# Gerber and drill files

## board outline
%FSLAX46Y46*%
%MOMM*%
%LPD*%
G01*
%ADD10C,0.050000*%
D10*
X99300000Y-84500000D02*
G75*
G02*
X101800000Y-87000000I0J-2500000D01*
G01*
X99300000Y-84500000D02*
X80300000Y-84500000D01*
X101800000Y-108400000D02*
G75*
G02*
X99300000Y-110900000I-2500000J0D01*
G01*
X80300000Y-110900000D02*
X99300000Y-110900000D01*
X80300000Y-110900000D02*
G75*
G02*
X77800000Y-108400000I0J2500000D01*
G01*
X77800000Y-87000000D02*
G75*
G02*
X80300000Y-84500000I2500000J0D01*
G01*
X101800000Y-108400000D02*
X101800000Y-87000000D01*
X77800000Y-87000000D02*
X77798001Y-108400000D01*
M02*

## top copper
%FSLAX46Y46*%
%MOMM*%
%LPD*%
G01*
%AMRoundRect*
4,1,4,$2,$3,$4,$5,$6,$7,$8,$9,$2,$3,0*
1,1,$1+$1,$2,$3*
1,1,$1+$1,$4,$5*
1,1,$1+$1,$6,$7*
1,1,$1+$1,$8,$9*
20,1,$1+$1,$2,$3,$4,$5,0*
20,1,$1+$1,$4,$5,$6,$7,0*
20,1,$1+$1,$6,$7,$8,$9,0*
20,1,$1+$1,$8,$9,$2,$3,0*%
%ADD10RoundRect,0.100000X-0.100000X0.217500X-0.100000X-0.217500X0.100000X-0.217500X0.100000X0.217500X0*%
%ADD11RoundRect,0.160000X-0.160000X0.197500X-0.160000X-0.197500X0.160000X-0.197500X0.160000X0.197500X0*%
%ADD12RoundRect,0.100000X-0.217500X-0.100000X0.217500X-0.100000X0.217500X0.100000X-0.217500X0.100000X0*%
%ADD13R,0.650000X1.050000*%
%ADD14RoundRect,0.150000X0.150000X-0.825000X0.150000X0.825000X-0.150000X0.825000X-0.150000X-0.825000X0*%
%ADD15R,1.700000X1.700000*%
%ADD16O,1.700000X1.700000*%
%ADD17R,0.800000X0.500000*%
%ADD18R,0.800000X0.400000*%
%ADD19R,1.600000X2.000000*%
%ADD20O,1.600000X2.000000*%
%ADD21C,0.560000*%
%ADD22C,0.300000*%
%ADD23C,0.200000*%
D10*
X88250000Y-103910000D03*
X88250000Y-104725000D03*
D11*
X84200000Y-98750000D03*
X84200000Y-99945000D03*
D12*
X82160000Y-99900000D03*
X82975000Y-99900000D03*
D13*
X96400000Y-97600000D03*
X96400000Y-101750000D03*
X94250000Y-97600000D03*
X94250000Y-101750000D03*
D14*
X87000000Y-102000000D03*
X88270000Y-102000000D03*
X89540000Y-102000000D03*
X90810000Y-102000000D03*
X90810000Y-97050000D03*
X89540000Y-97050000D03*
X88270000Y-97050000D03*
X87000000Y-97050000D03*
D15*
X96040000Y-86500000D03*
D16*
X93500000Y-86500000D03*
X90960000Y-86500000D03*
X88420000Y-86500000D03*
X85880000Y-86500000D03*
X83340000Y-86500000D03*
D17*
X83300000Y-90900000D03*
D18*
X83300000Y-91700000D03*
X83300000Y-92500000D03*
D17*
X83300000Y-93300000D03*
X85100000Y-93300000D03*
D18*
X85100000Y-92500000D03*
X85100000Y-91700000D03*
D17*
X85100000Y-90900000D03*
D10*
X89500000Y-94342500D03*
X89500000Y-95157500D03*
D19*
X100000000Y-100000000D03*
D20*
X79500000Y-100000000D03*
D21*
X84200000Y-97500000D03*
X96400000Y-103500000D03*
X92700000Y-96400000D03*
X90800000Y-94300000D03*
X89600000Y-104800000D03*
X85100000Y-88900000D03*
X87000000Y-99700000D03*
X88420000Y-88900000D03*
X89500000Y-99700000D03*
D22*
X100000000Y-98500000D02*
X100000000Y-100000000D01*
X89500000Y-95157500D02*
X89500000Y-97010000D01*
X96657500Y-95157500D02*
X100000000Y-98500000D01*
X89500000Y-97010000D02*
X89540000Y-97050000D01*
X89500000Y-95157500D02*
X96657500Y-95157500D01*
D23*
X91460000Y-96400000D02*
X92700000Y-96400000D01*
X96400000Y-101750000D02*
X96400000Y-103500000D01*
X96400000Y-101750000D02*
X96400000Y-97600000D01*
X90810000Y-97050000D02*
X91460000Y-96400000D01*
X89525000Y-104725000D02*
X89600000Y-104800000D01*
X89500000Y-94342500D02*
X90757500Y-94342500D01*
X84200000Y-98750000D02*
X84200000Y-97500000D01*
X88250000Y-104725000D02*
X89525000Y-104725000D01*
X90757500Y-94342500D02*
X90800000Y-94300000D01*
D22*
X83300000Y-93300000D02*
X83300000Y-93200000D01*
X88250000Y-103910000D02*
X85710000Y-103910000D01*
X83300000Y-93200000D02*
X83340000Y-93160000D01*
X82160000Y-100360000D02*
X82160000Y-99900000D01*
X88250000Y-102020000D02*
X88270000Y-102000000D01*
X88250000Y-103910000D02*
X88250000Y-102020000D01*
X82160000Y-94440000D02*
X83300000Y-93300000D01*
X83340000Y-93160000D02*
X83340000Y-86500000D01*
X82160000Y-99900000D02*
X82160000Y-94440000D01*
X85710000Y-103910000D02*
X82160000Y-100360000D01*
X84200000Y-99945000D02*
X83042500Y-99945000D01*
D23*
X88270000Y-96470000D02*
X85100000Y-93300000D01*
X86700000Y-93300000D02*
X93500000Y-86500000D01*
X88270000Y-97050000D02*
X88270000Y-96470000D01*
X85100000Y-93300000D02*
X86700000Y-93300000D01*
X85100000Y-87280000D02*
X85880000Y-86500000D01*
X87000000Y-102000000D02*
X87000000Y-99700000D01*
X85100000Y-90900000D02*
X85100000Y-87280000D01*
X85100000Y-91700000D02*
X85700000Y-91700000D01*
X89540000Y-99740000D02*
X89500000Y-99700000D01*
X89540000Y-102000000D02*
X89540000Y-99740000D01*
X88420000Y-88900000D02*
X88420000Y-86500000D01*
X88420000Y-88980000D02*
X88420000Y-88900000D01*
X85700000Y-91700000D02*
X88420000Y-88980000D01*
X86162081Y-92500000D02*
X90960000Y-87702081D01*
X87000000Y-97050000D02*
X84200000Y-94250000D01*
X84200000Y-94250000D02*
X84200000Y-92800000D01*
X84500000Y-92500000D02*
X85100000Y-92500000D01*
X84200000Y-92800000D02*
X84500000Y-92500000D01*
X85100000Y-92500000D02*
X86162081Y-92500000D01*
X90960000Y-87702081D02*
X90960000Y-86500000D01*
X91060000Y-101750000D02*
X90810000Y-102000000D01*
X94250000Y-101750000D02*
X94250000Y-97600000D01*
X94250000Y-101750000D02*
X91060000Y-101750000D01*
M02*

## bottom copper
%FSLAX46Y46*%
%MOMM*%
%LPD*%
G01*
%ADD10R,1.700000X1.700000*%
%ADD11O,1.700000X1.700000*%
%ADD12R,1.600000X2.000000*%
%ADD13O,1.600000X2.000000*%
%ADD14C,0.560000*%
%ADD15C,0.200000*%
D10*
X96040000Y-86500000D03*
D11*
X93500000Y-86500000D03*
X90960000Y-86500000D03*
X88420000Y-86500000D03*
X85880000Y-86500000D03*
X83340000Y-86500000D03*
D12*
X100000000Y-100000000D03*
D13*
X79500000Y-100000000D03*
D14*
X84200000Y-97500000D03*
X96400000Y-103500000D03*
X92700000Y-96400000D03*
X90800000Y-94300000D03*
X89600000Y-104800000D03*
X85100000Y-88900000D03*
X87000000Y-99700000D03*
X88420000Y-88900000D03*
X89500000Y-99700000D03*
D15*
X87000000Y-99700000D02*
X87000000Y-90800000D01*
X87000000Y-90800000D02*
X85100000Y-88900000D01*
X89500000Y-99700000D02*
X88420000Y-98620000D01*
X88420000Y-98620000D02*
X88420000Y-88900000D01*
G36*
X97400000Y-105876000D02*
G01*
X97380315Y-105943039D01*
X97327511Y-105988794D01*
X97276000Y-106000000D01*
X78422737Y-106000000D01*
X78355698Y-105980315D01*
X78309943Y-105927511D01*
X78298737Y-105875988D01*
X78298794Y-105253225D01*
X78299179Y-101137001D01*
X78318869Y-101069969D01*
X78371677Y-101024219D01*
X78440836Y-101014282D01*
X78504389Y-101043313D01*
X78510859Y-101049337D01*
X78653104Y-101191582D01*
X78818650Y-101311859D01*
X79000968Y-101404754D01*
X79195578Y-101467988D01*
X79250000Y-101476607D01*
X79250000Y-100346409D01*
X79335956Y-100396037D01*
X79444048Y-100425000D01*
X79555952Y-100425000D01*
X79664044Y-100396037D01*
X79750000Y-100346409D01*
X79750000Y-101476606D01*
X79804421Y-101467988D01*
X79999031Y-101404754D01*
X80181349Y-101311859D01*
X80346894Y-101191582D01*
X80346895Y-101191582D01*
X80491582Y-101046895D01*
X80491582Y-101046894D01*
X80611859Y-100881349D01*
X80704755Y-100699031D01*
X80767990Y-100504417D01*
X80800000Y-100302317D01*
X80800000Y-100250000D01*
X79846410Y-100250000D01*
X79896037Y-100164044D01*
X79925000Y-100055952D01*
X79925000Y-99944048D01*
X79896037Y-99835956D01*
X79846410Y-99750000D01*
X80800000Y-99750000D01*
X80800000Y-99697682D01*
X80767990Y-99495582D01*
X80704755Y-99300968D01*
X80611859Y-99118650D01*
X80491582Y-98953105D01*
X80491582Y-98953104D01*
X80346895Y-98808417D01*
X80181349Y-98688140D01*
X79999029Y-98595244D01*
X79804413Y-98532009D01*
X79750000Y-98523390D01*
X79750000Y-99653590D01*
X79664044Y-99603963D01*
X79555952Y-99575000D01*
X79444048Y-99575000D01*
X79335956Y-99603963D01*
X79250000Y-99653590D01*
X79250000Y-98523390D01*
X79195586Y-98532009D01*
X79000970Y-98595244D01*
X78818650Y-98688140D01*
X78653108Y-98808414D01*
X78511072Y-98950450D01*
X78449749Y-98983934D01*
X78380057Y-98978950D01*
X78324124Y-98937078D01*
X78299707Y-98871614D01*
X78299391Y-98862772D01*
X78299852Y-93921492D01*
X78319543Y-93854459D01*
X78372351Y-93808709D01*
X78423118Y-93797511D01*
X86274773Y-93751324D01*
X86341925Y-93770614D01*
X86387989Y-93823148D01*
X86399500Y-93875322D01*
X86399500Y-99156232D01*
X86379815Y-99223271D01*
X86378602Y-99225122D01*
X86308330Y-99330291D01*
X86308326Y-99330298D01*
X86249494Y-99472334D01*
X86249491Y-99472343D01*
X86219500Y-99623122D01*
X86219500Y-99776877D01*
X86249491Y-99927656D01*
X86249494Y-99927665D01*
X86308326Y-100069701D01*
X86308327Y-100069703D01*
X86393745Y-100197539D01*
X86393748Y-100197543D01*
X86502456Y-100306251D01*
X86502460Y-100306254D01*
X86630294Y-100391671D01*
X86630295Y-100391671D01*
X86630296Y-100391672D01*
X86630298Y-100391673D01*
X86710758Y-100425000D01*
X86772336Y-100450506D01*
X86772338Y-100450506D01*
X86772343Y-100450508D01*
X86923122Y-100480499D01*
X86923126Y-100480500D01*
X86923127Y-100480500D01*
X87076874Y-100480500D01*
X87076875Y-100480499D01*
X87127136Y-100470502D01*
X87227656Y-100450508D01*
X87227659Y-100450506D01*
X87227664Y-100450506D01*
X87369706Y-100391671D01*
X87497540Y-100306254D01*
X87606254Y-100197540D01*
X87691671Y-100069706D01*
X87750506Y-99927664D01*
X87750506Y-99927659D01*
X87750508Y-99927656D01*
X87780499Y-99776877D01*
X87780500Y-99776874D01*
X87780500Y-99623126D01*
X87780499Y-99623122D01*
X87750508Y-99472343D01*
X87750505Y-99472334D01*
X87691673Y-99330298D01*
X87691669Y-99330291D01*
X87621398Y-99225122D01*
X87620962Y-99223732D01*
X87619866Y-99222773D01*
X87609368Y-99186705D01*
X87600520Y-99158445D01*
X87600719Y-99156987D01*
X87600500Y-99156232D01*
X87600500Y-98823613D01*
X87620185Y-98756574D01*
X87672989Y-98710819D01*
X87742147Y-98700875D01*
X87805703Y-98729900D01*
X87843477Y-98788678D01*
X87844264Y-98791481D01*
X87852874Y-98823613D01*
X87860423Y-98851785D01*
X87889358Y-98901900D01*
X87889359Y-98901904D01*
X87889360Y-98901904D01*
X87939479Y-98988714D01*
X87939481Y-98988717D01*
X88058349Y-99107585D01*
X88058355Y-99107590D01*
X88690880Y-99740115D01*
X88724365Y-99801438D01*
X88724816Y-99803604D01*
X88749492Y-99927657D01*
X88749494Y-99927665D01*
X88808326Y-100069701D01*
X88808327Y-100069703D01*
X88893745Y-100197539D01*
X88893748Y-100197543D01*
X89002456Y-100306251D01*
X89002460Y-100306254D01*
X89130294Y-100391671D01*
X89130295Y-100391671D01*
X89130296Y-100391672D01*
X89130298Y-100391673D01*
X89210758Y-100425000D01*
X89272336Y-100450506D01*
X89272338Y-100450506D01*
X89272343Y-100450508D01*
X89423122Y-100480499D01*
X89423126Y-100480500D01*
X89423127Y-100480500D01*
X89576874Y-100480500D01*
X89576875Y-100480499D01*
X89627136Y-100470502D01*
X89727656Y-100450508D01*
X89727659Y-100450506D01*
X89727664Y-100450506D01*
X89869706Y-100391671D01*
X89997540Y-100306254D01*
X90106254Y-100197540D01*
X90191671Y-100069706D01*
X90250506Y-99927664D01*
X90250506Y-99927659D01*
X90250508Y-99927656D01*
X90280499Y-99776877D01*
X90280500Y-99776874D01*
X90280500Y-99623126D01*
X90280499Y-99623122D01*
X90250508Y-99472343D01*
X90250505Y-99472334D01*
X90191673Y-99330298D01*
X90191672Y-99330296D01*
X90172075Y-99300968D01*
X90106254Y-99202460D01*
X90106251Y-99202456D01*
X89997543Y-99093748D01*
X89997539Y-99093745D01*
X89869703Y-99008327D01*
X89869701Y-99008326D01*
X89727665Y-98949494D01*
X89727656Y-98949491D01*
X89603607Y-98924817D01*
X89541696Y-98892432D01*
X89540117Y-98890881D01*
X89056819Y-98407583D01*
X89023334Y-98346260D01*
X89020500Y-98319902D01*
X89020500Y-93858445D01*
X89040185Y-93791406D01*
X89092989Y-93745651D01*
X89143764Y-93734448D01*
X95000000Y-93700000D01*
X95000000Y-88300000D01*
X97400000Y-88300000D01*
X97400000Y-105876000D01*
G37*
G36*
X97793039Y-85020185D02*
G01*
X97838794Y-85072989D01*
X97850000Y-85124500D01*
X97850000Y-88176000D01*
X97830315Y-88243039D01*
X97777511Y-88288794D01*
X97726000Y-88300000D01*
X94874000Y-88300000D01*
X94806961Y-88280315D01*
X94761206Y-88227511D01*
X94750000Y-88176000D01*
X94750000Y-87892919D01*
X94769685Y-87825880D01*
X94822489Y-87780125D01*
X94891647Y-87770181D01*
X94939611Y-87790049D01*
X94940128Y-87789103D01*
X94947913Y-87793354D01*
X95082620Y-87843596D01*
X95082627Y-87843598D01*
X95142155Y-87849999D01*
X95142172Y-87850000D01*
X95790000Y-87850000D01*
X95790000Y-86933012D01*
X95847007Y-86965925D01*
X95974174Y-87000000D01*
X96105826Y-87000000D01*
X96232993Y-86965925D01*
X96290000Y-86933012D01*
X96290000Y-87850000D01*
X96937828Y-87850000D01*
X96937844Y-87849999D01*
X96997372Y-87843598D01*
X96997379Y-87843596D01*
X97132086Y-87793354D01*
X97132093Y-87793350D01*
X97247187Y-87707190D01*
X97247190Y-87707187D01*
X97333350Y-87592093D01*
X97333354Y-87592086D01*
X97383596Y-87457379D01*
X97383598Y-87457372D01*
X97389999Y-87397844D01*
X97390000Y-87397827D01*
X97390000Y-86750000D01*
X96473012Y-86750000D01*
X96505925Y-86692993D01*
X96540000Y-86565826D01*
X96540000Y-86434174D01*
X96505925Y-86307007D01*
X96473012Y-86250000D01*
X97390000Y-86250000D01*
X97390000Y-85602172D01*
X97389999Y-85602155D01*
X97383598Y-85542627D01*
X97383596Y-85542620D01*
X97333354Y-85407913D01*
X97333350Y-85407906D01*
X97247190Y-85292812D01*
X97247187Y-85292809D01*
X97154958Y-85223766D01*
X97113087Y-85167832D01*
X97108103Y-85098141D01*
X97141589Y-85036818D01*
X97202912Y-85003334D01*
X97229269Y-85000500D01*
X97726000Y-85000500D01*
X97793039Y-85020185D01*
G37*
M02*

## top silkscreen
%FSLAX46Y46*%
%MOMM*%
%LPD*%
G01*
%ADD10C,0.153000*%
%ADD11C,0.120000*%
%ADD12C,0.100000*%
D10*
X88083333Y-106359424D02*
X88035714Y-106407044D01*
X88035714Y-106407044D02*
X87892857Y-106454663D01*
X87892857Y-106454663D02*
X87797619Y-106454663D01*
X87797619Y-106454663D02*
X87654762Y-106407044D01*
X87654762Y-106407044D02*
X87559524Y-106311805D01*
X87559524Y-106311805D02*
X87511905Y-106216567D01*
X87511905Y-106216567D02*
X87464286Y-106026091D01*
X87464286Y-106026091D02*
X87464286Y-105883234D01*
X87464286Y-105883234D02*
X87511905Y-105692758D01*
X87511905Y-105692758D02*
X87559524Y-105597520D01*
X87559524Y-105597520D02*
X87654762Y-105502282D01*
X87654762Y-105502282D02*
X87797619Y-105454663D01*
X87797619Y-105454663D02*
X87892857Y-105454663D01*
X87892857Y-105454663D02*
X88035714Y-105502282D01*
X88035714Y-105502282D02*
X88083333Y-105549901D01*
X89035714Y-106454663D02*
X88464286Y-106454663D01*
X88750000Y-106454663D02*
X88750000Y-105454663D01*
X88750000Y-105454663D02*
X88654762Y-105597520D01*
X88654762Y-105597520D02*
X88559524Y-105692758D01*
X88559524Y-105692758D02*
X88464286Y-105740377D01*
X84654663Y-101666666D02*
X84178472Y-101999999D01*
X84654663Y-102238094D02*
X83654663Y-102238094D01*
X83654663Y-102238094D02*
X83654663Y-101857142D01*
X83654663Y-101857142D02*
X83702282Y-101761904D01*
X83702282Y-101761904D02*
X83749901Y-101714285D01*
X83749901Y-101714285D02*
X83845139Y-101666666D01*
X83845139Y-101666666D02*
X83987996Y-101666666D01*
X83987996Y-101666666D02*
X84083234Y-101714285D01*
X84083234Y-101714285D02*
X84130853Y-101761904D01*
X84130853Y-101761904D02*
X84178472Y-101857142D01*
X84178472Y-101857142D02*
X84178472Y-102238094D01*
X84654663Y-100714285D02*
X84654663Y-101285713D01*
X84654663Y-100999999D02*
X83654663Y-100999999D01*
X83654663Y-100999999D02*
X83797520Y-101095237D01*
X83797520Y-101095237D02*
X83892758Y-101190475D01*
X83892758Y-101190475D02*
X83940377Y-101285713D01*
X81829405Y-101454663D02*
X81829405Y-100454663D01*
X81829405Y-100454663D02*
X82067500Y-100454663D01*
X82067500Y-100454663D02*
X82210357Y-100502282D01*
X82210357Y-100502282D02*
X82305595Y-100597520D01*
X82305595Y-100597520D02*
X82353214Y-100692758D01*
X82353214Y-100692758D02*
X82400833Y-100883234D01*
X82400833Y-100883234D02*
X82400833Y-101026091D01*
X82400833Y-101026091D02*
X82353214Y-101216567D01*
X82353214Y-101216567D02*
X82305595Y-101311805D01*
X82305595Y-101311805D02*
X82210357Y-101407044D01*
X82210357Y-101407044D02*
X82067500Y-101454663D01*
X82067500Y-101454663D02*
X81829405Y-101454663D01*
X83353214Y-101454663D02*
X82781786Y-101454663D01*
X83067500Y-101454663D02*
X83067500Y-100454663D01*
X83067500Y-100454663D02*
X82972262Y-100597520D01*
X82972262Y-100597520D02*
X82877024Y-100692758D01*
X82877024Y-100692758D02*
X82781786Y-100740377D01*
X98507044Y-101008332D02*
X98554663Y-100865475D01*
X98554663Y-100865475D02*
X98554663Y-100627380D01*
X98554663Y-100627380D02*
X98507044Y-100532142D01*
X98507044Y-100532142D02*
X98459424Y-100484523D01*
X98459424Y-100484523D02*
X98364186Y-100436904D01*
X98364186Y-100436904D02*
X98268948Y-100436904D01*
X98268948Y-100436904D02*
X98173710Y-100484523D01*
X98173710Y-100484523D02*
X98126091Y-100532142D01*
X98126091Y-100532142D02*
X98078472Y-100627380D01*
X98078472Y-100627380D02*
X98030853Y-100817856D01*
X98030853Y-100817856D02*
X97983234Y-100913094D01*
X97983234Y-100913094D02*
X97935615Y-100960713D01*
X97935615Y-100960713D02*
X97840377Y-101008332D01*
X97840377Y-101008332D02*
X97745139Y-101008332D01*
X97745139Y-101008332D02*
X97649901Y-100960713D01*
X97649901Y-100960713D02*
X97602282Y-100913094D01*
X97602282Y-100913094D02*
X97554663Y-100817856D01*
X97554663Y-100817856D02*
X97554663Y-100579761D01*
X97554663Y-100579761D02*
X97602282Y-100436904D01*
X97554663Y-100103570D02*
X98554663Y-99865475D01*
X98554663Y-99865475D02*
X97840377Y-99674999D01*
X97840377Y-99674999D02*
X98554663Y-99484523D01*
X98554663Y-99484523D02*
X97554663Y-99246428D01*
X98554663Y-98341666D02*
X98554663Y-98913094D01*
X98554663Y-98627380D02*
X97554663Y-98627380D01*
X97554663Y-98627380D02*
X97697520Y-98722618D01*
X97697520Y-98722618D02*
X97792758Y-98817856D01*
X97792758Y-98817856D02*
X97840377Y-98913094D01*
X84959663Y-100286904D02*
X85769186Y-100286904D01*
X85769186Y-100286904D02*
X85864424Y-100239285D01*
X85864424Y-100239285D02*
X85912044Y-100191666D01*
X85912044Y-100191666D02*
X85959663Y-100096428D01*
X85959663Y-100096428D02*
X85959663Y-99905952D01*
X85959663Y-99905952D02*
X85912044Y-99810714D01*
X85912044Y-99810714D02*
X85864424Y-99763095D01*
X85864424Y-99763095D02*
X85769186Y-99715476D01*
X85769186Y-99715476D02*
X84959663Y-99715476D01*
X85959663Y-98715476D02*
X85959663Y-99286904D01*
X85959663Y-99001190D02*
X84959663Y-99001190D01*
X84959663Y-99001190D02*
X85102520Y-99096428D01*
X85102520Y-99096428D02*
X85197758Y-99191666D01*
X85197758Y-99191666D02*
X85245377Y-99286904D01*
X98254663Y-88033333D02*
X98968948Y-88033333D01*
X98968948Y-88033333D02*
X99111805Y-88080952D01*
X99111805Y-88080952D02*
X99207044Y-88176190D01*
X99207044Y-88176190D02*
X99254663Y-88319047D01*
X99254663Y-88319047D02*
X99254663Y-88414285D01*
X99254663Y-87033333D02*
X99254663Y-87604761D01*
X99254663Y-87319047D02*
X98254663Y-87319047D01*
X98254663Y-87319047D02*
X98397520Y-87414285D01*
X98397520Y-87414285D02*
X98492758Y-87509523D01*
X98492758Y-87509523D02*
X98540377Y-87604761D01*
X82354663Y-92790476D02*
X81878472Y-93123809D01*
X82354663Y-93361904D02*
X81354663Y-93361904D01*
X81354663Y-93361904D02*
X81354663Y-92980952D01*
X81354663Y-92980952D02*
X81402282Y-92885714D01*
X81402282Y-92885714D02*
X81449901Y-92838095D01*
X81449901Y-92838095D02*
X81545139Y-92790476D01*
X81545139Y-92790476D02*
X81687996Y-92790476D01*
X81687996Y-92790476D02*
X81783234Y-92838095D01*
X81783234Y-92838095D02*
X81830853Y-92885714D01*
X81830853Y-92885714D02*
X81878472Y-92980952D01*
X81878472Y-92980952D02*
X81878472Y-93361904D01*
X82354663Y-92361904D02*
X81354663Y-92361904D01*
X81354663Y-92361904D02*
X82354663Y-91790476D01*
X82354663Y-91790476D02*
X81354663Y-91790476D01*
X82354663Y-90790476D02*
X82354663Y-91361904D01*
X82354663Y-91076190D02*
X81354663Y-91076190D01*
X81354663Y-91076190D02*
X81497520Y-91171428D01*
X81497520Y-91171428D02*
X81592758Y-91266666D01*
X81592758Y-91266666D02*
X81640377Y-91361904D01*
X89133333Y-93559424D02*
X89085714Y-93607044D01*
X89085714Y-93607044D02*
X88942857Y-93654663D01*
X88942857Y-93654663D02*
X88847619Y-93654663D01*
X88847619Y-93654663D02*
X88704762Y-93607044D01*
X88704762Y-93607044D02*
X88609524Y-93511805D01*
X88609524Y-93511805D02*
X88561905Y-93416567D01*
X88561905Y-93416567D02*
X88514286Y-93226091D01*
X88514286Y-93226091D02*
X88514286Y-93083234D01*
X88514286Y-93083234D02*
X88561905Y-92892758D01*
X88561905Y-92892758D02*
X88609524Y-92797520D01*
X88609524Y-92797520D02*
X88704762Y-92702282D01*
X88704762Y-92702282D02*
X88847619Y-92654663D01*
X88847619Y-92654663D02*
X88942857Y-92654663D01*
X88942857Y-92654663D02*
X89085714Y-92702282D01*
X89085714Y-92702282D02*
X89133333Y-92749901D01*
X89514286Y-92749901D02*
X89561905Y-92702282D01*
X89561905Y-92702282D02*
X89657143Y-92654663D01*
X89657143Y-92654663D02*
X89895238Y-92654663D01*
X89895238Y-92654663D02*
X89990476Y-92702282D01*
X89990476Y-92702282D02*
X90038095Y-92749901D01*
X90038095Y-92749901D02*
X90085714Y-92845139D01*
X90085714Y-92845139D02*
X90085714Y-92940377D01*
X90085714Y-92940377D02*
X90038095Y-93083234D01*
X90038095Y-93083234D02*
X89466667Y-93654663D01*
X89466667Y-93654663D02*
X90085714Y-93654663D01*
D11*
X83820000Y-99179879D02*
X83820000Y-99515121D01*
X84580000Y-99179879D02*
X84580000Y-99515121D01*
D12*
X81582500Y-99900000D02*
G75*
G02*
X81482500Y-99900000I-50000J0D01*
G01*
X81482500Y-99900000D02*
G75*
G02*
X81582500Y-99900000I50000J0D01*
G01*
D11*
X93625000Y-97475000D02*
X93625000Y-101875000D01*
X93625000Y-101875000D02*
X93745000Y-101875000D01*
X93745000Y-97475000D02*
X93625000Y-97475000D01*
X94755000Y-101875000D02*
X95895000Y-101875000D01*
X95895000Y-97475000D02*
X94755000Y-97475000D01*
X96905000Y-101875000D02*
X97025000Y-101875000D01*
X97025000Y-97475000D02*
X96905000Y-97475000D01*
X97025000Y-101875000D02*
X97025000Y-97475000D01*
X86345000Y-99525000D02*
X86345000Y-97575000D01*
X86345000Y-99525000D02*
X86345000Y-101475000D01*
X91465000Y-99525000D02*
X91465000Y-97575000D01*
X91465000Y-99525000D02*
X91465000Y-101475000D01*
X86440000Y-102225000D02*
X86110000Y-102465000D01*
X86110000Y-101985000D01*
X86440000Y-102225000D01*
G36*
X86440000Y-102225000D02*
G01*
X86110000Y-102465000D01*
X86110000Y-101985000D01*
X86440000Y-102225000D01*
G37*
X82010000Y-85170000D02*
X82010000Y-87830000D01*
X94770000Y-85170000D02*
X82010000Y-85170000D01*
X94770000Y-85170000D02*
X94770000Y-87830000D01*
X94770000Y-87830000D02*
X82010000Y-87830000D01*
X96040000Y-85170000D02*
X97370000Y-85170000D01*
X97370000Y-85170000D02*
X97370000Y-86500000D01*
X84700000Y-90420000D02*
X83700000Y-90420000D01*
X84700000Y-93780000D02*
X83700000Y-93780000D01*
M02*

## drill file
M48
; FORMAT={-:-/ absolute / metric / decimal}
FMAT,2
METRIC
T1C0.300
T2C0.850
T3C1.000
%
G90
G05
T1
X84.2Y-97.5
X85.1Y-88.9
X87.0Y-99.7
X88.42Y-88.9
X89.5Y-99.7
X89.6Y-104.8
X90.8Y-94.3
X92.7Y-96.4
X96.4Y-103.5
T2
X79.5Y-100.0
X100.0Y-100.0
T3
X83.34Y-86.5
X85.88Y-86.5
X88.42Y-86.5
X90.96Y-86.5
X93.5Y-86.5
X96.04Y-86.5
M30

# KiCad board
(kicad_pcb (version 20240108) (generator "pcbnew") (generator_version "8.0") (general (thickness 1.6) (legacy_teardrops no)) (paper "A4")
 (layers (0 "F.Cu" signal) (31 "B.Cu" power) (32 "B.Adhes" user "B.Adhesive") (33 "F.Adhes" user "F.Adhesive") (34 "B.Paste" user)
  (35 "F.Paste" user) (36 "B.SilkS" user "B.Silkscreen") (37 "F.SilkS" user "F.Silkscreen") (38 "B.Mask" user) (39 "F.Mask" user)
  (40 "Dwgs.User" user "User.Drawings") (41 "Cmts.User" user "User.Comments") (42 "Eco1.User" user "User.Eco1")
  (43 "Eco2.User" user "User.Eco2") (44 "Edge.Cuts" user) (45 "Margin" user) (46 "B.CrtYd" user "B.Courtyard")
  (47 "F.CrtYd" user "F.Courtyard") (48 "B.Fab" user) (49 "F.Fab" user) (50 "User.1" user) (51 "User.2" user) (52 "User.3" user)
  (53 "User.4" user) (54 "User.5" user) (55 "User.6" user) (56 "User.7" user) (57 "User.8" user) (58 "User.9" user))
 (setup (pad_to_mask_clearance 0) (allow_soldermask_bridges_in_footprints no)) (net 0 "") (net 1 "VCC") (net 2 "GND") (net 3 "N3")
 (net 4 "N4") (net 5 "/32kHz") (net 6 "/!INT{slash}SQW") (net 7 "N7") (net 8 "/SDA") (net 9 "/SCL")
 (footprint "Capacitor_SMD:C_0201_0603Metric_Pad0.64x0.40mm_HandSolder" (layer "F.Cu") (at 88.25 104.3175 -90)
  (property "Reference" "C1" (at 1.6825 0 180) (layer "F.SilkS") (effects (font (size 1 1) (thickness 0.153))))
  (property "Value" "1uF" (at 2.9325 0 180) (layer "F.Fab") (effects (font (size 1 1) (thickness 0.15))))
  (pad "" smd roundrect (at -0.4325 0 270) (size 0.458 0.36) (layers "F.Paste") (roundrect_rratio 0.25))
  (pad "" smd roundrect (at 0.4325 0 270) (size 0.458 0.36) (layers "F.Paste") (roundrect_rratio 0.25))
  (pad "1" smd roundrect (at -0.4075 0 270) (size 0.635 0.4) (layers "F.Cu" "F.Mask") (roundrect_rratio 0.25) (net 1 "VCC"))
  (pad "2" smd roundrect (at 0.4075 0 270) (size 0.635 0.4) (layers "F.Cu" "F.Mask") (roundrect_rratio 0.25) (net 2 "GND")))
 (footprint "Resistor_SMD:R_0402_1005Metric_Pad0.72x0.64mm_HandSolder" (layer "F.Cu") (at 84.2 99.3475 -90)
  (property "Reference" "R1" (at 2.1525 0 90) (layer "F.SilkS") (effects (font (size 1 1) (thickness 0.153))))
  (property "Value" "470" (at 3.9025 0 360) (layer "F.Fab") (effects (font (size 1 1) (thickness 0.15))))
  (fp_line (start -0.167621 0.38) (end 0.167621 0.38) (stroke (width 0.12) (type solid)) (layer "F.SilkS"))
  (fp_line (start -0.167621 -0.38) (end 0.167621 -0.38) (stroke (width 0.12) (type solid)) (layer "F.SilkS"))
  (pad "1" smd roundrect (at -0.5975 0 270) (size 0.715 0.64) (layers "F.Cu" "F.Paste" "F.Mask") (roundrect_rratio 0.25) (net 2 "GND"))
  (pad "2" smd roundrect (at 0.5975 0 270) (size 0.715 0.64) (layers "F.Cu" "F.Paste" "F.Mask") (roundrect_rratio 0.25) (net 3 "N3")))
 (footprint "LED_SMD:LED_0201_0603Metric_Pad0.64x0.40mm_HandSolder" (layer "F.Cu") (at 82.5675 99.9)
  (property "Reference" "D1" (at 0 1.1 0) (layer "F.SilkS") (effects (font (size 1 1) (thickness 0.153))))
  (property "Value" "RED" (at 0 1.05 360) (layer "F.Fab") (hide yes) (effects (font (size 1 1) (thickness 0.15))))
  (fp_circle (center -1.035 0) (end -0.985 0) (stroke (width 0.1) (type solid)) (fill none) (layer "F.SilkS"))
  (pad "" smd roundrect (at -0.4325 0) (size 0.458 0.36) (layers "F.Paste") (roundrect_rratio 0.25))
  (pad "" smd roundrect (at 0.4325 0) (size 0.458 0.36) (layers "F.Paste") (roundrect_rratio 0.25))
  (pad "1" smd roundrect (at -0.4075 0) (size 0.635 0.4) (layers "F.Cu" "F.Mask") (roundrect_rratio 0.25) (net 1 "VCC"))
  (pad "2" smd roundrect (at 0.4075 0) (size 0.635 0.4) (layers "F.Cu" "F.Mask") (roundrect_rratio 0.25) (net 3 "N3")))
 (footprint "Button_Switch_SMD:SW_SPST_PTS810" (layer "F.Cu") (at 95.325 99.675 -90)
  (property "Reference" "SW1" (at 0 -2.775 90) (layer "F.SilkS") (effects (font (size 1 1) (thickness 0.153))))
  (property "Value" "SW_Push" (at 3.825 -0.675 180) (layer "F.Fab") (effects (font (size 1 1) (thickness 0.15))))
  (fp_line (start -2.2 1.7) (end 2.2 1.7) (stroke (width 0.12) (type solid)) (layer "F.SilkS"))
  (fp_line (start 2.2 1.7) (end 2.2 1.58) (stroke (width 0.12) (type solid)) (layer "F.SilkS"))
  (fp_line (start -2.2 1.58) (end -2.2 1.7) (stroke (width 0.12) (type solid)) (layer "F.SilkS"))
  (fp_line (start 2.2 0.57) (end 2.2 -0.57) (stroke (width 0.12) (type solid)) (layer "F.SilkS"))
  (fp_line (start -2.2 -0.57) (end -2.2 0.57) (stroke (width 0.12) (type solid)) (layer "F.SilkS"))
  (fp_line (start 2.2 -1.58) (end 2.2 -1.7) (stroke (width 0.12) (type solid)) (layer "F.SilkS"))
  (fp_line (start -2.2 -1.7) (end -2.2 -1.58) (stroke (width 0.12) (type solid)) (layer "F.SilkS"))
  (fp_line (start 2.2 -1.7) (end -2.2 -1.7) (stroke (width 0.12) (type solid)) (layer "F.SilkS"))
  (pad "1" smd rect (at -2.075 -1.075 270) (size 1.05 0.65) (layers "F.Cu" "F.Paste" "F.Mask") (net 2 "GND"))
  (pad "1" smd rect (at 2.075 -1.075 270) (size 1.05 0.65) (layers "F.Cu" "F.Paste" "F.Mask") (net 2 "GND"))
  (pad "2" smd rect (at -2.075 1.075 270) (size 1.05 0.65) (layers "F.Cu" "F.Paste" "F.Mask") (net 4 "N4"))
  (pad "2" smd rect (at 2.075 1.075 270) (size 1.05 0.65) (layers "F.Cu" "F.Paste" "F.Mask") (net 4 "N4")))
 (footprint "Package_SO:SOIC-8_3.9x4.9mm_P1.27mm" (layer "F.Cu") (at 88.905 99.525 90)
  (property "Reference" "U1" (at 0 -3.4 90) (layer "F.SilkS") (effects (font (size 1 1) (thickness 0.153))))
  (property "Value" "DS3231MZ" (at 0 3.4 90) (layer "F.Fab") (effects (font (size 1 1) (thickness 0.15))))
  (fp_line (start 0 -2.56) (end 1.95 -2.56) (stroke (width 0.12) (type solid)) (layer "F.SilkS"))
  (fp_line (start 0 -2.56) (end -1.95 -2.56) (stroke (width 0.12) (type solid)) (layer "F.SilkS"))
  (fp_line (start 0 2.56) (end 1.95 2.56) (stroke (width 0.12) (type solid)) (layer "F.SilkS"))
  (fp_line (start 0 2.56) (end -1.95 2.56) (stroke (width 0.12) (type solid)) (layer "F.SilkS"))
  (fp_poly
   (pts (xy -2.7 -2.465) (xy -2.94 -2.795) (xy -2.46 -2.795) (xy -2.7 -2.465)) (stroke (width 0.12) (type solid)) (fill solid)
   (layer "F.SilkS"))
  (pad "1" smd roundrect (at -2.475 -1.905 90) (size 1.95 0.6) (layers "F.Cu" "F.Paste" "F.Mask") (roundrect_rratio 0.25) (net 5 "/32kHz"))
  (pad "2" smd roundrect (at -2.475 -0.635 90) (size 1.95 0.6) (layers "F.Cu" "F.Paste" "F.Mask") (roundrect_rratio 0.25) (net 1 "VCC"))
  (pad "3" smd roundrect (at -2.475 0.635 90) (size 1.95 0.6) (layers "F.Cu" "F.Paste" "F.Mask") (roundrect_rratio 0.25)
   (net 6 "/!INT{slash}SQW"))
  (pad "4" smd roundrect (at -2.475 1.905 90) (size 1.95 0.6) (layers "F.Cu" "F.Paste" "F.Mask") (roundrect_rratio 0.25) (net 4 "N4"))
  (pad "5" smd roundrect (at 2.475 1.905 90) (size 1.95 0.6) (layers "F.Cu" "F.Paste" "F.Mask") (roundrect_rratio 0.25) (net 2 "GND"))
  (pad "6" smd roundrect (at 2.475 0.635 90) (size 1.95 0.6) (layers "F.Cu" "F.Paste" "F.Mask") (roundrect_rratio 0.25) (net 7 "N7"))
  (pad "7" smd roundrect (at 2.475 -0.635 90) (size 1.95 0.6) (layers "F.Cu" "F.Paste" "F.Mask") (roundrect_rratio 0.25) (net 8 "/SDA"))
  (pad "8" smd roundrect (at 2.475 -1.905 90) (size 1.95 0.6) (layers "F.Cu" "F.Paste" "F.Mask") (roundrect_rratio 0.25) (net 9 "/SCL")))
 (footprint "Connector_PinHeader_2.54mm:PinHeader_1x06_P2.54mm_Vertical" (layer "F.Cu") (at 96.04 86.5 -90)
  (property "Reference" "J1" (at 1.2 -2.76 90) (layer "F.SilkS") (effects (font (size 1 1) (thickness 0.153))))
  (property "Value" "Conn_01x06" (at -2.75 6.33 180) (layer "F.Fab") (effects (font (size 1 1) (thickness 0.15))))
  (fp_line (start -1.33 14.03) (end 1.33 14.03) (stroke (width 0.12) (type solid)) (layer "F.SilkS"))
  (fp_line (start -1.33 1.27) (end -1.33 14.03) (stroke (width 0.12) (type solid)) (layer "F.SilkS"))
  (fp_line (start -1.33 1.27) (end 1.33 1.27) (stroke (width 0.12) (type solid)) (layer "F.SilkS"))
  (fp_line (start 1.33 1.27) (end 1.33 14.03) (stroke (width 0.12) (type solid)) (layer "F.SilkS"))
  (fp_line (start -1.33 0) (end -1.33 -1.33) (stroke (width 0.12) (type solid)) (layer "F.SilkS"))
  (fp_line (start -1.33 -1.33) (end 0 -1.33) (stroke (width 0.12) (type solid)) (layer "F.SilkS"))
  (pad "1" thru_hole rect (at 0 0 270) (size 1.7 1.7) (drill 1) (layers "*.Cu" "*.Mask") (remove_unused_layers no) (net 2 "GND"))
  (pad "2" thru_hole oval (at 0 2.54 270) (size 1.7 1.7) (drill 1) (layers "*.Cu" "*.Mask") (remove_unused_layers no) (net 8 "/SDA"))
  (pad "3" thru_hole oval (at 0 5.08 270) (size 1.7 1.7) (drill 1) (layers "*.Cu" "*.Mask") (remove_unused_layers no) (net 9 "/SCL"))
  (pad "4" thru_hole oval (at 0 7.62 270) (size 1.7 1.7) (drill 1) (layers "*.Cu" "*.Mask") (remove_unused_layers no)
   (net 6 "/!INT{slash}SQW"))
  (pad "5" thru_hole oval (at 0 10.16 270) (size 1.7 1.7) (drill 1) (layers "*.Cu" "*.Mask") (remove_unused_layers no) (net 5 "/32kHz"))
  (pad "6" thru_hole oval (at 0 12.7 270) (size 1.7 1.7) (drill 1) (layers "*.Cu" "*.Mask") (remove_unused_layers no) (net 1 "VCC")))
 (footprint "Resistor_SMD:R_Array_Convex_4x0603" (layer "F.Cu") (at 84.2 92.1)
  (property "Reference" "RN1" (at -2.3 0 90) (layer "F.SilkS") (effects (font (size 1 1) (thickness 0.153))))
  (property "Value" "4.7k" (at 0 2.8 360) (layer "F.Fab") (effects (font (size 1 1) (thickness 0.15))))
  (fp_line (start 0.5 -1.68) (end -0.5 -1.68) (stroke (width 0.12) (type solid)) (layer "F.SilkS"))
  (fp_line (start 0.5 1.68) (end -0.5 1.68) (stroke (width 0.12) (type solid)) (layer "F.SilkS"))
  (pad "1" smd rect (at -0.9 -1.2) (size 0.8 0.5) (layers "F.Cu" "F.Paste" "F.Mask") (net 1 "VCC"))
  (pad "2" smd rect (at -0.9 -0.4) (size 0.8 0.4) (layers "F.Cu" "F.Paste" "F.Mask") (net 1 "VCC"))
  (pad "3" smd rect (at -0.9 0.4) (size 0.8 0.4) (layers "F.Cu" "F.Paste" "F.Mask") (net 1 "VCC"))
  (pad "4" smd rect (at -0.9 1.2) (size 0.8 0.5) (layers "F.Cu" "F.Paste" "F.Mask") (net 1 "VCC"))
  (pad "5" smd rect (at 0.9 1.2) (size 0.8 0.5) (layers "F.Cu" "F.Paste" "F.Mask") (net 8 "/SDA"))
  (pad "6" smd rect (at 0.9 0.4) (size 0.8 0.4) (layers "F.Cu" "F.Paste" "F.Mask") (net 9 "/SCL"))
  (pad "7" smd rect (at 0.9 -0.4) (size 0.8 0.4) (layers "F.Cu" "F.Paste" "F.Mask") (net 6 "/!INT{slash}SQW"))
  (pad "8" smd rect (at 0.9 -1.2) (size 0.8 0.5) (layers "F.Cu" "F.Paste" "F.Mask") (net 5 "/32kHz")))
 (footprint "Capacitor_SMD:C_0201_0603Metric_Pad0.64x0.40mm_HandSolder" (layer "F.Cu") (at 89.5 94.75 -90)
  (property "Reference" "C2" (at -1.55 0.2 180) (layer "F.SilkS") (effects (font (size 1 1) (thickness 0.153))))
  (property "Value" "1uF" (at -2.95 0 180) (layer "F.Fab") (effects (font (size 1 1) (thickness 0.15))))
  (pad "" smd roundrect (at -0.4325 0 270) (size 0.458 0.36) (layers "F.Paste") (roundrect_rratio 0.25))
  (pad "" smd roundrect (at 0.4325 0 270) (size 0.458 0.36) (layers "F.Paste") (roundrect_rratio 0.25))
  (pad "1" smd roundrect (at -0.4075 0 270) (size 0.635 0.4) (layers "F.Cu" "F.Mask") (roundrect_rratio 0.25) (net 2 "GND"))
  (pad "2" smd roundrect (at 0.4075 0 270) (size 0.635 0.4) (layers "F.Cu" "F.Mask") (roundrect_rratio 0.25) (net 7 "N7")))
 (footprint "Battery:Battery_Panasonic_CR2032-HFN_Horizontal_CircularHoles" (layer "B.Cu") (at 100 100 180)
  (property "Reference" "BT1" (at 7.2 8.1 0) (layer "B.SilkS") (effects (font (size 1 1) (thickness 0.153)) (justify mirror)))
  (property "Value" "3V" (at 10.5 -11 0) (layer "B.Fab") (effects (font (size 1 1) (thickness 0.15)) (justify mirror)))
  (pad "1" thru_hole rect (at 0 0 180) (size 1.6 2) (drill 0.85) (layers "*.Cu" "*.Mask") (remove_unused_layers no) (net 7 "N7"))
  (pad "2" thru_hole oval (at 20.5 0 180) (size 1.6 2) (drill 0.85) (layers "*.Cu" "*.Mask") (remove_unused_layers no) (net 2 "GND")))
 (gr_arc (start 99.3 84.5) (mid 101.067767 85.232233) (end 101.8 87) (stroke (width 0.05) (type default)) (layer "Edge.Cuts"))
 (gr_line (start 99.3 84.5) (end 80.3 84.5) (stroke (width 0.05) (type default)) (layer "Edge.Cuts"))
 (gr_arc (start 101.8 108.4) (mid 101.067767 110.167767) (end 99.3 110.9) (stroke (width 0.05) (type default)) (layer "Edge.Cuts"))
 (gr_line (start 80.3 110.9) (end 99.3 110.9) (stroke (width 0.05) (type default)) (layer "Edge.Cuts"))
 (gr_arc (start 80.3 110.9) (mid 78.532233 110.167767) (end 77.8 108.4) (stroke (width 0.05) (type default)) (layer "Edge.Cuts"))
 (gr_arc (start 77.8 87) (mid 78.532233 85.232233) (end 80.3 84.5) (stroke (width 0.05) (type default)) (layer "Edge.Cuts"))
 (gr_line (start 101.8 108.4) (end 101.8 87) (stroke (width 0.05) (type default)) (layer "Edge.Cuts"))
 (gr_line (start 77.8 87) (end 77.798001 108.4) (stroke (width 0.05) (type default)) (layer "Edge.Cuts"))
 (segment (start 100 98.5) (end 100 100) (width 0.3) (layer "F.Cu") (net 7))
 (segment (start 89.5 95.1575) (end 89.5 97.01) (width 0.3) (layer "F.Cu") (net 7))
 (segment (start 96.6575 95.1575) (end 100 98.5) (width 0.3) (layer "F.Cu") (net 7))
 (segment (start 89.5 97.01) (end 89.54 97.05) (width 0.3) (layer "F.Cu") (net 7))
 (segment (start 89.5 95.1575) (end 96.6575 95.1575) (width 0.3) (layer "F.Cu") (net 7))
 (segment (start 91.46 96.4) (end 92.7 96.4) (width 0.2) (layer "F.Cu") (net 2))
 (segment (start 96.4 101.75) (end 96.4 103.5) (width 0.2) (layer "F.Cu") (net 2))
 (segment (start 96.4 101.75) (end 96.4 97.6) (width 0.2) (layer "F.Cu") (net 2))
 (segment (start 90.81 97.05) (end 91.46 96.4) (width 0.2) (layer "F.Cu") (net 2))
 (segment (start 89.525 104.725) (end 89.6 104.8) (width 0.2) (layer "F.Cu") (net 2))
 (segment (start 89.5 94.3425) (end 90.7575 94.3425) (width 0.2) (layer "F.Cu") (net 2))
 (segment (start 84.2 98.75) (end 84.2 97.5) (width 0.2) (layer "F.Cu") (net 2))
 (segment (start 88.25 104.725) (end 89.525 104.725) (width 0.2) (layer "F.Cu") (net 2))
 (segment (start 90.7575 94.3425) (end 90.8 94.3) (width 0.2) (layer "F.Cu") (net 2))
 (via (at 84.2 97.5) (size 0.56) (drill 0.3) (layers "F.Cu" "B.Cu") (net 2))
 (via (at 96.4 103.5) (size 0.56) (drill 0.3) (layers "F.Cu" "B.Cu") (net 2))
 (via (at 92.7 96.4) (size 0.56) (drill 0.3) (layers "F.Cu" "B.Cu") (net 2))
 (via (at 90.8 94.3) (size 0.56) (drill 0.3) (layers "F.Cu" "B.Cu") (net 2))
 (via (at 89.6 104.8) (size 0.56) (drill 0.3) (layers "F.Cu" "B.Cu") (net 2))
 (segment (start 83.3 93.3) (end 83.3 93.2) (width 0.3) (layer "F.Cu") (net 1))
 (segment (start 88.25 103.91) (end 85.71 103.91) (width 0.3) (layer "F.Cu") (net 1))
 (segment (start 83.3 93.2) (end 83.34 93.16) (width 0.3) (layer "F.Cu") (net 1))
 (segment (start 82.16 100.36) (end 82.16 99.9) (width 0.3) (layer "F.Cu") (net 1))
 (segment (start 88.25 102.02) (end 88.27 102) (width 0.3) (layer "F.Cu") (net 1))
 (segment (start 88.25 103.91) (end 88.25 102.02) (width 0.3) (layer "F.Cu") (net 1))
 (segment (start 82.16 94.44) (end 83.3 93.3) (width 0.3) (layer "F.Cu") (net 1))
 (segment (start 83.34 93.16) (end 83.34 86.5) (width 0.3) (layer "F.Cu") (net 1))
 (segment (start 82.16 99.9) (end 82.16 94.44) (width 0.3) (layer "F.Cu") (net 1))
 (segment (start 85.71 103.91) (end 82.16 100.36) (width 0.3) (layer "F.Cu") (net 1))
 (segment (start 84.2 99.945) (end 83.0425 99.945) (width 0.3) (layer "F.Cu") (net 3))
 (segment (start 88.27 96.47) (end 85.1 93.3) (width 0.2) (layer "F.Cu") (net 8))
 (segment (start 86.7 93.3) (end 93.5 86.5) (width 0.2) (layer "F.Cu") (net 8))
 (segment (start 88.27 97.05) (end 88.27 96.47) (width 0.2) (layer "F.Cu") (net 8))
 (segment (start 85.1 93.3) (end 86.7 93.3) (width 0.2) (layer "F.Cu") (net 8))
 (segment (start 85.1 87.28) (end 85.88 86.5) (width 0.2) (layer "F.Cu") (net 5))
 (segment (start 87 102) (end 87 99.7) (width 0.2) (layer "F.Cu") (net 5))
 (segment (start 85.1 90.9) (end 85.1 87.28) (width 0.2) (layer "F.Cu") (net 5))
 (via (at 85.1 88.9) (size 0.56) (drill 0.3) (layers "F.Cu" "B.Cu") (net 5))
 (via (at 87 99.7) (size 0.56) (drill 0.3) (layers "F.Cu" "B.Cu") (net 5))
 (segment (start 87 99.7) (end 87 90.8) (width 0.2) (layer "B.Cu") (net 5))
 (segment (start 87 90.8) (end 85.1 88.9) (width 0.2) (layer "B.Cu") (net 5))
 (segment (start 85.1 91.7) (end 85.7 91.7) (width 0.2) (layer "F.Cu") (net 6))
 (segment (start 89.54 99.74) (end 89.5 99.7) (width 0.2) (layer "F.Cu") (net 6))
 (segment (start 89.54 102) (end 89.54 99.74) (width 0.2) (layer "F.Cu") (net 6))
 (segment (start 88.42 88.9) (end 88.42 86.5) (width 0.2) (layer "F.Cu") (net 6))
 (segment (start 88.42 88.98) (end 88.42 88.9) (width 0.2) (layer "F.Cu") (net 6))
 (segment (start 85.7 91.7) (end 88.42 88.98) (width 0.2) (layer "F.Cu") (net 6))
 (via (at 88.42 88.9) (size 0.56) (drill 0.3) (layers "F.Cu" "B.Cu") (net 6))
 (via (at 89.5 99.7) (size 0.56) (drill 0.3) (layers "F.Cu" "B.Cu") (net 6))
 (segment (start 89.5 99.7) (end 88.42 98.62) (width 0.2) (layer "B.Cu") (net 6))
 (segment (start 88.42 98.62) (end 88.42 88.9) (width 0.2) (layer "B.Cu") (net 6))
 (segment (start 86.162081 92.5) (end 90.96 87.702081) (width 0.2) (layer "F.Cu") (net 9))
 (segment (start 87 97.05) (end 84.2 94.25) (width 0.2) (layer "F.Cu") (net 9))
 (segment (start 84.2 94.25) (end 84.2 92.8) (width 0.2) (layer "F.Cu") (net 9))
 (segment (start 84.5 92.5) (end 85.1 92.5) (width 0.2) (layer "F.Cu") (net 9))
 (segment (start 84.2 92.8) (end 84.5 92.5) (width 0.2) (layer "F.Cu") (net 9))
 (segment (start 85.1 92.5) (end 86.162081 92.5) (width 0.2) (layer "F.Cu") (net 9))
 (segment (start 90.96 87.702081) (end 90.96 86.5) (width 0.2) (layer "F.Cu") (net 9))
 (segment (start 91.06 101.75) (end 90.81 102) (width 0.2) (layer "F.Cu") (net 4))
 (segment (start 94.25 101.75) (end 94.25 97.6) (width 0.2) (layer "F.Cu") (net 4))
 (segment (start 94.25 101.75) (end 91.06 101.75) (width 0.2) (layer "F.Cu") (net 4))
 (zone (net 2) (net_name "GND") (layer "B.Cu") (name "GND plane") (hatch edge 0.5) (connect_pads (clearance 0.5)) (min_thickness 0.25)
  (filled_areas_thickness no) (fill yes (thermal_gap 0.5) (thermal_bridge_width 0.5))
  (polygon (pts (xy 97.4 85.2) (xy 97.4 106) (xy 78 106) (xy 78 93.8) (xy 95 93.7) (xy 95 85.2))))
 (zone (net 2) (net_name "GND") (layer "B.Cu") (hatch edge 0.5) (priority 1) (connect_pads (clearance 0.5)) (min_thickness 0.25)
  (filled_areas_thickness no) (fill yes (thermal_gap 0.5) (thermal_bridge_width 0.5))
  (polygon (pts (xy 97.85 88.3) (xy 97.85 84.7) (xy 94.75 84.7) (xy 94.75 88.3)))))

